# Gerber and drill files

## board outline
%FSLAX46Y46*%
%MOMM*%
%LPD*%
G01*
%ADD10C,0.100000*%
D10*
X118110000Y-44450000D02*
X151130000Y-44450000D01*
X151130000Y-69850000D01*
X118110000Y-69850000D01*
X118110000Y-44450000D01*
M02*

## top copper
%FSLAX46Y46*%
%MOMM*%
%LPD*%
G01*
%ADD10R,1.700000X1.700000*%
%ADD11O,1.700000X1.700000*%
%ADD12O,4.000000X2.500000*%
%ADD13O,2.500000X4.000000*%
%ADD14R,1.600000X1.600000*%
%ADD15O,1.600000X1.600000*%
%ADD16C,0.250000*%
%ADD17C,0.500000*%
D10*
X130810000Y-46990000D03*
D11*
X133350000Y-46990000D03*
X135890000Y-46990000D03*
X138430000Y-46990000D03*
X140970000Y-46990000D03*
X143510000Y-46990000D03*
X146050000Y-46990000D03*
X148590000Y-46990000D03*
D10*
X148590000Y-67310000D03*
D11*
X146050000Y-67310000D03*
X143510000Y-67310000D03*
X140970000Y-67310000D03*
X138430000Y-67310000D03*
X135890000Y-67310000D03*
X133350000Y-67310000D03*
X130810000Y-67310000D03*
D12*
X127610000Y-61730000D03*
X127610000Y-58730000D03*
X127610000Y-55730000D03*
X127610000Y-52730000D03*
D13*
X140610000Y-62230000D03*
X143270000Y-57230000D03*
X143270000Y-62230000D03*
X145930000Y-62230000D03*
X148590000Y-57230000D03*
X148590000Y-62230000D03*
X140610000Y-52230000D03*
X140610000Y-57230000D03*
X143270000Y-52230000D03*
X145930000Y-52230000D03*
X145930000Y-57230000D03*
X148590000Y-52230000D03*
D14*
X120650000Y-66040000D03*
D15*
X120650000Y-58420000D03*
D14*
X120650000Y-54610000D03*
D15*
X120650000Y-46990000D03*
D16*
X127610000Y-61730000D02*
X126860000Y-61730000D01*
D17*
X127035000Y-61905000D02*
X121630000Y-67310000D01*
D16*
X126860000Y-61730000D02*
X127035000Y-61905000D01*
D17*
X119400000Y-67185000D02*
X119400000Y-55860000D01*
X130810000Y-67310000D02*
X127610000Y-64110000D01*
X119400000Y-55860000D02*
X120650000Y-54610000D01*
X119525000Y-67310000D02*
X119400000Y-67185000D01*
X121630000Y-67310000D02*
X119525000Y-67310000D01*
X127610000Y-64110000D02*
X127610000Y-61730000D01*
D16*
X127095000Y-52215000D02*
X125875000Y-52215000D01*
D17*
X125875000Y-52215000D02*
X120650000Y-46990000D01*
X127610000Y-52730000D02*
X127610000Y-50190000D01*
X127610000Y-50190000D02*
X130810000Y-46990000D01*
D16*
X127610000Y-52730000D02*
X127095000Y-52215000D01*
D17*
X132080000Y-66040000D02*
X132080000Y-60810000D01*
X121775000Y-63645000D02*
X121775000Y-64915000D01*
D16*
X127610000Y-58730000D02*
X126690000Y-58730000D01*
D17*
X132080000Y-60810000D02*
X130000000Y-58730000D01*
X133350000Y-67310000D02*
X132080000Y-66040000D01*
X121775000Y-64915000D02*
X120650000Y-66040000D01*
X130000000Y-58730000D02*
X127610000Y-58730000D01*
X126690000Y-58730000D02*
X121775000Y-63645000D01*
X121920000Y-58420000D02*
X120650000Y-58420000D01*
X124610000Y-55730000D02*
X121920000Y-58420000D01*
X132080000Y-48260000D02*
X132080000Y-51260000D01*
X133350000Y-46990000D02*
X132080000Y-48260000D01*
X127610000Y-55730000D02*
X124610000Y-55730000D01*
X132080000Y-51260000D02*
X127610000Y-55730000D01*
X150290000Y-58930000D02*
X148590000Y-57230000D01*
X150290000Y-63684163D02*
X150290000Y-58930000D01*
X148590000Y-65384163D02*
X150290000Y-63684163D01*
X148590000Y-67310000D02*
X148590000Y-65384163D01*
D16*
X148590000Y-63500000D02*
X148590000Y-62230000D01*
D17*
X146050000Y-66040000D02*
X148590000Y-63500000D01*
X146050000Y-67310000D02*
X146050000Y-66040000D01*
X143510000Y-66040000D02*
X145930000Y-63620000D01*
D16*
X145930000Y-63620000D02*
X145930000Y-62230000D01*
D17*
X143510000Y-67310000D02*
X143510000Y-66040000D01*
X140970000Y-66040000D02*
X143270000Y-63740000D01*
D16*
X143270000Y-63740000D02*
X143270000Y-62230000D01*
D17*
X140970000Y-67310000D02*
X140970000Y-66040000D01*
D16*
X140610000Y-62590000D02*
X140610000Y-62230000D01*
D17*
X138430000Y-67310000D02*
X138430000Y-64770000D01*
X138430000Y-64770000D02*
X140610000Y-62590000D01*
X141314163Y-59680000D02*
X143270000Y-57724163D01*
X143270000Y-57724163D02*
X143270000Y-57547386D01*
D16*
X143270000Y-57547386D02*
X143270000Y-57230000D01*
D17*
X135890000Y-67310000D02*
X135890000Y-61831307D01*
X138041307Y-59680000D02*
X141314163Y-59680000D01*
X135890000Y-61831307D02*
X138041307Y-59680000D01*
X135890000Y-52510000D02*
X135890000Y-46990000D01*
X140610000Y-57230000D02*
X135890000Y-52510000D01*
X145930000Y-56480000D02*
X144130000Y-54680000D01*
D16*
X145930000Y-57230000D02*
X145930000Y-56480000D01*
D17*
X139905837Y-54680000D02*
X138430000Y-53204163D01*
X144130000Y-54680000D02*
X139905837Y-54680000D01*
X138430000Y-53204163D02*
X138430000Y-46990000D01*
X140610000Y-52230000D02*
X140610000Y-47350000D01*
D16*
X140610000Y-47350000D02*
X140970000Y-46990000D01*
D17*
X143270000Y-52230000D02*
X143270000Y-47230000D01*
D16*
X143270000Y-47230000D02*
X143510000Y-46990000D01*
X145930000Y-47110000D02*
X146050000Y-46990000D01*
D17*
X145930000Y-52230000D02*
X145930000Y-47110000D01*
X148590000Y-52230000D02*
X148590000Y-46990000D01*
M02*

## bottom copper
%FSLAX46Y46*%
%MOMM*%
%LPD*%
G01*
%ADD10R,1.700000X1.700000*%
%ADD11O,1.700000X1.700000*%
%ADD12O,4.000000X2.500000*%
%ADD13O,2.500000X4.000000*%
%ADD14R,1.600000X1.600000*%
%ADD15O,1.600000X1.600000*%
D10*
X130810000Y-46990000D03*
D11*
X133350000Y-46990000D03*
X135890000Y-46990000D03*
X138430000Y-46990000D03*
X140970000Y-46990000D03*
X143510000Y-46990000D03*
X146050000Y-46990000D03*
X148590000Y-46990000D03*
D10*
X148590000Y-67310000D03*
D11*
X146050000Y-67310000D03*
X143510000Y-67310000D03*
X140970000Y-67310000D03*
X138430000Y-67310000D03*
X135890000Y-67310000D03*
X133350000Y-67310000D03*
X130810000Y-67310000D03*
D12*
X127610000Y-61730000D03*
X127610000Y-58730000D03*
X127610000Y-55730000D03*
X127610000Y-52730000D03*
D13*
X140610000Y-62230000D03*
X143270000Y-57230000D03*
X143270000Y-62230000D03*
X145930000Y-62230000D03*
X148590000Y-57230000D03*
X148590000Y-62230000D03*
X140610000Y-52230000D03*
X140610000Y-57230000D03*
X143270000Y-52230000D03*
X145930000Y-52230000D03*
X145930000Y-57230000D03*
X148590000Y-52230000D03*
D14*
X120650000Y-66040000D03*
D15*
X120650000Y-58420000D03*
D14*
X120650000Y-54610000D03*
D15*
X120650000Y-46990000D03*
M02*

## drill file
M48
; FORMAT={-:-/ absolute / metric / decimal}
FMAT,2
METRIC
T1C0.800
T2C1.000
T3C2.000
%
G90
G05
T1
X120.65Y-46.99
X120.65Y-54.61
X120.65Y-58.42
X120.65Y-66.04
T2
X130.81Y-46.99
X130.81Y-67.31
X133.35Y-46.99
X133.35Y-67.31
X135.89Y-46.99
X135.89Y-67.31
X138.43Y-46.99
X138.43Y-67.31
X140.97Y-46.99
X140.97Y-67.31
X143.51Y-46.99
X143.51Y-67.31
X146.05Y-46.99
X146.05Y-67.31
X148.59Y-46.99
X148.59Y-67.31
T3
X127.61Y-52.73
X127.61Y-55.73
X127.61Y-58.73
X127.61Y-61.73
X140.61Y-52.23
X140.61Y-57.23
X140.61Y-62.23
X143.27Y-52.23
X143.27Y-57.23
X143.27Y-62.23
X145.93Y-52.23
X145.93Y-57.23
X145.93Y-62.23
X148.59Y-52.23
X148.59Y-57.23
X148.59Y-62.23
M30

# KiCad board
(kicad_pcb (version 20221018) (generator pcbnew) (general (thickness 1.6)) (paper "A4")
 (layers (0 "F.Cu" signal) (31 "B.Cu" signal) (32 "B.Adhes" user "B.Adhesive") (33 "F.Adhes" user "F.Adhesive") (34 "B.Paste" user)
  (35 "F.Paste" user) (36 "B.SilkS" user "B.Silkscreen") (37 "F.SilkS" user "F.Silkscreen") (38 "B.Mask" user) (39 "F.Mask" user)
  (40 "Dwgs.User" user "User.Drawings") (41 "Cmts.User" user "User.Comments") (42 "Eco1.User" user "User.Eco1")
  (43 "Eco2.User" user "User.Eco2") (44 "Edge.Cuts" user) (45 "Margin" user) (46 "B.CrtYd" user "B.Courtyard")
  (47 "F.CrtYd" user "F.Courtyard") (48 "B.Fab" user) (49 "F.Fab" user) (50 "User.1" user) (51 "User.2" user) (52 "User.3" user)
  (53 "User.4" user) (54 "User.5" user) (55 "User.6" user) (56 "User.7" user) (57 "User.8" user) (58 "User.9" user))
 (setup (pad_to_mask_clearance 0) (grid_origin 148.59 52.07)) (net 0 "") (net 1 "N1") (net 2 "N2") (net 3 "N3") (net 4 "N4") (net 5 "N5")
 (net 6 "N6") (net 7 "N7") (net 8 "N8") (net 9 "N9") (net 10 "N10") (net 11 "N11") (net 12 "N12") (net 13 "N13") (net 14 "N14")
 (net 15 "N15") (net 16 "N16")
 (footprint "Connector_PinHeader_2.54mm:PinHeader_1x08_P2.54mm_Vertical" (layer "F.Cu") (at 130.81 46.99 90)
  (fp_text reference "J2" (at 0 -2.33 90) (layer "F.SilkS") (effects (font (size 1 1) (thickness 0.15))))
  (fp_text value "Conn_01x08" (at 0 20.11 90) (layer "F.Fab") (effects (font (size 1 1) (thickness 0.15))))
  (pad "1" thru_hole rect (at 0 0 90) (size 1.7 1.7) (drill 1) (layers "*.Cu" "*.Mask") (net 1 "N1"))
  (pad "2" thru_hole oval (at 0 2.54 90) (size 1.7 1.7) (drill 1) (layers "*.Cu" "*.Mask") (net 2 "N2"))
  (pad "3" thru_hole oval (at 0 5.08 90) (size 1.7 1.7) (drill 1) (layers "*.Cu" "*.Mask") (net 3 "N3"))
  (pad "4" thru_hole oval (at 0 7.62 90) (size 1.7 1.7) (drill 1) (layers "*.Cu" "*.Mask") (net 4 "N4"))
  (pad "5" thru_hole oval (at 0 10.16 90) (size 1.7 1.7) (drill 1) (layers "*.Cu" "*.Mask") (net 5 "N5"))
  (pad "6" thru_hole oval (at 0 12.7 90) (size 1.7 1.7) (drill 1) (layers "*.Cu" "*.Mask") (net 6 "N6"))
  (pad "7" thru_hole oval (at 0 15.24 90) (size 1.7 1.7) (drill 1) (layers "*.Cu" "*.Mask") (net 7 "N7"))
  (pad "8" thru_hole oval (at 0 17.78 90) (size 1.7 1.7) (drill 1) (layers "*.Cu" "*.Mask") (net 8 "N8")))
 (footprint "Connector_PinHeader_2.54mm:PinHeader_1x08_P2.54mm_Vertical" (layer "F.Cu") (at 148.59 67.31 -90)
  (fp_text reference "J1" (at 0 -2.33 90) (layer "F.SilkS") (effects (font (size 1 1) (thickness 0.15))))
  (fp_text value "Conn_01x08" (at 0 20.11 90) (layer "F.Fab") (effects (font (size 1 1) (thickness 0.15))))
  (pad "1" thru_hole rect (at 0 0 270) (size 1.7 1.7) (drill 1) (layers "*.Cu" "*.Mask") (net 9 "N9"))
  (pad "2" thru_hole oval (at 0 2.54 270) (size 1.7 1.7) (drill 1) (layers "*.Cu" "*.Mask") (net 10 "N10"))
  (pad "3" thru_hole oval (at 0 5.08 270) (size 1.7 1.7) (drill 1) (layers "*.Cu" "*.Mask") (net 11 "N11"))
  (pad "4" thru_hole oval (at 0 7.62 270) (size 1.7 1.7) (drill 1) (layers "*.Cu" "*.Mask") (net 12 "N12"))
  (pad "5" thru_hole oval (at 0 10.16 270) (size 1.7 1.7) (drill 1) (layers "*.Cu" "*.Mask") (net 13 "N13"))
  (pad "6" thru_hole oval (at 0 12.7 270) (size 1.7 1.7) (drill 1) (layers "*.Cu" "*.Mask") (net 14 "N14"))
  (pad "7" thru_hole oval (at 0 15.24 270) (size 1.7 1.7) (drill 1) (layers "*.Cu" "*.Mask") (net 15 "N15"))
  (pad "8" thru_hole oval (at 0 17.78 270) (size 1.7 1.7) (drill 1) (layers "*.Cu" "*.Mask") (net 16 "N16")))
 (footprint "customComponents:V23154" (layer "F.Cu") (at 140.61 57.23)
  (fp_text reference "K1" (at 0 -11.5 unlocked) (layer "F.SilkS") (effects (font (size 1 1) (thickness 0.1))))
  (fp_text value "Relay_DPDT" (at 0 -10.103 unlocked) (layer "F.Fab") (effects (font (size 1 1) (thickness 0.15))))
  (pad "1" thru_hole oval (at -13 4.5) (size 4 2.5) (drill 2) (layers "*.Cu" "*.Mask") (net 16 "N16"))
  (pad "2" thru_hole oval (at -13 1.5) (size 4 2.5) (drill 2) (layers "*.Cu" "*.Mask") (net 15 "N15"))
  (pad "3" thru_hole oval (at -13 -1.5) (size 4 2.5) (drill 2) (layers "*.Cu" "*.Mask") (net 2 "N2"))
  (pad "4" thru_hole oval (at -13 -4.5) (size 4 2.5) (drill 2) (layers "*.Cu" "*.Mask") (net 1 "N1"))
  (pad "5" thru_hole oval (at 0 5 90) (size 4 2.5) (drill 2) (layers "*.Cu" "*.Mask") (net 13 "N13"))
  (pad "6" thru_hole oval (at 2.66 0 90) (size 4 2.5) (drill 2) (layers "*.Cu" "*.Mask") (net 14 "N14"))
  (pad "7" thru_hole oval (at 2.66 5 90) (size 4 2.5) (drill 2) (layers "*.Cu" "*.Mask") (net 12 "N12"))
  (pad "8" thru_hole oval (at 5.32 5 90) (size 4 2.5) (drill 2) (layers "*.Cu" "*.Mask") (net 11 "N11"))
  (pad "9" thru_hole oval (at 7.98 0 90) (size 4 2.5) (drill 2) (layers "*.Cu" "*.Mask") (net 9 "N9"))
  (pad "10" thru_hole oval (at 7.98 5 90) (size 4 2.5) (drill 2) (layers "*.Cu" "*.Mask") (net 10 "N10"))
  (pad "11" thru_hole oval (at 0 -5 90) (size 4 2.5) (drill 2) (layers "*.Cu" "*.Mask") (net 5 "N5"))
  (pad "12" thru_hole oval (at 0 0 90) (size 4 2.5) (drill 2) (layers "*.Cu" "*.Mask") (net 3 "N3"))
  (pad "13" thru_hole oval (at 2.66 -5 90) (size 4 2.5) (drill 2) (layers "*.Cu" "*.Mask") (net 6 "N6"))
  (pad "14" thru_hole oval (at 5.32 -5 90) (size 4 2.5) (drill 2) (layers "*.Cu" "*.Mask") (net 7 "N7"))
  (pad "15" thru_hole oval (at 5.32 0 90) (size 4 2.5) (drill 2) (layers "*.Cu" "*.Mask") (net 4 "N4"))
  (pad "16" thru_hole oval (at 7.98 -5 90) (size 4 2.5) (drill 2) (layers "*.Cu" "*.Mask") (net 8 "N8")))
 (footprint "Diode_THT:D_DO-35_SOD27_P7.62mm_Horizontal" (layer "F.Cu") (at 120.65 66.04 90)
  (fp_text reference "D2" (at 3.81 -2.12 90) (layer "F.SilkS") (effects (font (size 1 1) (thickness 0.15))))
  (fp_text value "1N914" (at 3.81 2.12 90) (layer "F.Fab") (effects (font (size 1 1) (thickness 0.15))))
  (pad "1" thru_hole rect (at 0 0 90) (size 1.6 1.6) (drill 0.8) (layers "*.Cu" "*.Mask") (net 15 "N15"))
  (pad "2" thru_hole oval (at 7.62 0 90) (size 1.6 1.6) (drill 0.8) (layers "*.Cu" "*.Mask") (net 2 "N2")))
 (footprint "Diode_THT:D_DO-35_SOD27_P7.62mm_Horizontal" (layer "F.Cu") (at 120.65 54.61 90)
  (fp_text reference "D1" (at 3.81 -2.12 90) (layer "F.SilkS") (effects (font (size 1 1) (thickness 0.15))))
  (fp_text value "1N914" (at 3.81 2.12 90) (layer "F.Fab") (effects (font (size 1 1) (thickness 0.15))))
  (pad "1" thru_hole rect (at 0 0 90) (size 1.6 1.6) (drill 0.8) (layers "*.Cu" "*.Mask") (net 16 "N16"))
  (pad "2" thru_hole oval (at 7.62 0 90) (size 1.6 1.6) (drill 0.8) (layers "*.Cu" "*.Mask") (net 1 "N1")))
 (gr_rect (start 118.11 44.45) (end 151.13 69.85) (stroke (width 0.1) (type default)) (fill none) (layer "Edge.Cuts"))
 (segment (start 127.61 61.73) (end 126.86 61.73) (width 0.25) (layer "F.Cu") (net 16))
 (segment (start 127.035 61.905) (end 121.63 67.31) (width 0.5) (layer "F.Cu") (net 16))
 (segment (start 126.86 61.73) (end 127.035 61.905) (width 0.25) (layer "F.Cu") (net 16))
 (segment (start 119.4 67.185) (end 119.4 55.86) (width 0.5) (layer "F.Cu") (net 16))
 (segment (start 130.81 67.31) (end 127.61 64.11) (width 0.5) (layer "F.Cu") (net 16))
 (segment (start 119.4 55.86) (end 120.65 54.61) (width 0.5) (layer "F.Cu") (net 16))
 (segment (start 119.525 67.31) (end 119.4 67.185) (width 0.5) (layer "F.Cu") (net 16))
 (segment (start 121.63 67.31) (end 119.525 67.31) (width 0.5) (layer "F.Cu") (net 16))
 (segment (start 127.61 64.11) (end 127.61 61.73) (width 0.5) (layer "F.Cu") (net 16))
 (segment (start 127.095 52.215) (end 125.875 52.215) (width 0.25) (layer "F.Cu") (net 1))
 (segment (start 125.875 52.215) (end 120.65 46.99) (width 0.5) (layer "F.Cu") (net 1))
 (segment (start 127.61 52.73) (end 127.61 50.19) (width 0.5) (layer "F.Cu") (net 1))
 (segment (start 127.61 50.19) (end 130.81 46.99) (width 0.5) (layer "F.Cu") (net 1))
 (segment (start 127.61 52.73) (end 127.095 52.215) (width 0.25) (layer "F.Cu") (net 1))
 (segment (start 132.08 66.04) (end 132.08 60.81) (width 0.5) (layer "F.Cu") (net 15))
 (segment (start 121.775 63.645) (end 121.775 64.915) (width 0.5) (layer "F.Cu") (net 15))
 (segment (start 127.61 58.73) (end 126.69 58.73) (width 0.25) (layer "F.Cu") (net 15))
 (segment (start 132.08 60.81) (end 130 58.73) (width 0.5) (layer "F.Cu") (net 15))
 (segment (start 133.35 67.31) (end 132.08 66.04) (width 0.5) (layer "F.Cu") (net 15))
 (segment (start 121.775 64.915) (end 120.65 66.04) (width 0.5) (layer "F.Cu") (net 15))
 (segment (start 130 58.73) (end 127.61 58.73) (width 0.5) (layer "F.Cu") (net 15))
 (segment (start 126.69 58.73) (end 121.775 63.645) (width 0.5) (layer "F.Cu") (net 15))
 (segment (start 121.92 58.42) (end 120.65 58.42) (width 0.5) (layer "F.Cu") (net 2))
 (segment (start 124.61 55.73) (end 121.92 58.42) (width 0.5) (layer "F.Cu") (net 2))
 (segment (start 132.08 48.26) (end 132.08 51.26) (width 0.5) (layer "F.Cu") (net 2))
 (segment (start 133.35 46.99) (end 132.08 48.26) (width 0.5) (layer "F.Cu") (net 2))
 (segment (start 127.61 55.73) (end 124.61 55.73) (width 0.5) (layer "F.Cu") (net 2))
 (segment (start 132.08 51.26) (end 127.61 55.73) (width 0.5) (layer "F.Cu") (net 2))
 (segment (start 150.29 58.93) (end 148.59 57.23) (width 0.5) (layer "F.Cu") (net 9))
 (segment (start 150.29 63.684163) (end 150.29 58.93) (width 0.5) (layer "F.Cu") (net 9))
 (segment (start 148.59 65.384163) (end 150.29 63.684163) (width 0.5) (layer "F.Cu") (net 9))
 (segment (start 148.59 67.31) (end 148.59 65.384163) (width 0.5) (layer "F.Cu") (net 9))
 (segment (start 148.59 63.5) (end 148.59 62.23) (width 0.25) (layer "F.Cu") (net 10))
 (segment (start 146.05 66.04) (end 148.59 63.5) (width 0.5) (layer "F.Cu") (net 10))
 (segment (start 146.05 67.31) (end 146.05 66.04) (width 0.5) (layer "F.Cu") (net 10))
 (segment (start 143.51 66.04) (end 145.93 63.62) (width 0.5) (layer "F.Cu") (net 11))
 (segment (start 145.93 63.62) (end 145.93 62.23) (width 0.25) (layer "F.Cu") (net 11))
 (segment (start 143.51 67.31) (end 143.51 66.04) (width 0.5) (layer "F.Cu") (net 11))
 (segment (start 140.97 66.04) (end 143.27 63.74) (width 0.5) (layer "F.Cu") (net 12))
 (segment (start 143.27 63.74) (end 143.27 62.23) (width 0.25) (layer "F.Cu") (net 12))
 (segment (start 140.97 67.31) (end 140.97 66.04) (width 0.5) (layer "F.Cu") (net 12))
 (segment (start 140.61 62.59) (end 140.61 62.23) (width 0.25) (layer "F.Cu") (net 13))
 (segment (start 138.43 67.31) (end 138.43 64.77) (width 0.5) (layer "F.Cu") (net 13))
 (segment (start 138.43 64.77) (end 140.61 62.59) (width 0.5) (layer "F.Cu") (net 13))
 (segment (start 141.314163 59.68) (end 143.27 57.724163) (width 0.5) (layer "F.Cu") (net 14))
 (segment (start 143.27 57.724163) (end 143.27 57.547386) (width 0.5) (layer "F.Cu") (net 14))
 (segment (start 143.27 57.547386) (end 143.27 57.23) (width 0.25) (layer "F.Cu") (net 14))
 (segment (start 135.89 67.31) (end 135.89 61.831307) (width 0.5) (layer "F.Cu") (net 14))
 (segment (start 138.041307 59.68) (end 141.314163 59.68) (width 0.5) (layer "F.Cu") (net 14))
 (segment (start 135.89 61.831307) (end 138.041307 59.68) (width 0.5) (layer "F.Cu") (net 14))
 (segment (start 135.89 52.51) (end 135.89 46.99) (width 0.5) (layer "F.Cu") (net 3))
 (segment (start 140.61 57.23) (end 135.89 52.51) (width 0.5) (layer "F.Cu") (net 3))
 (segment (start 145.93 56.48) (end 144.13 54.68) (width 0.5) (layer "F.Cu") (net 4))
 (segment (start 145.93 57.23) (end 145.93 56.48) (width 0.25) (layer "F.Cu") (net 4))
 (segment (start 139.905837 54.68) (end 138.43 53.204163) (width 0.5) (layer "F.Cu") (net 4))
 (segment (start 144.13 54.68) (end 139.905837 54.68) (width 0.5) (layer "F.Cu") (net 4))
 (segment (start 138.43 53.204163) (end 138.43 46.99) (width 0.5) (layer "F.Cu") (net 4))
 (segment (start 140.61 52.23) (end 140.61 47.35) (width 0.5) (layer "F.Cu") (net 5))
 (segment (start 140.61 47.35) (end 140.97 46.99) (width 0.25) (layer "F.Cu") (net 5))
 (segment (start 143.27 52.23) (end 143.27 47.23) (width 0.5) (layer "F.Cu") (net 6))
 (segment (start 143.27 47.23) (end 143.51 46.99) (width 0.25) (layer "F.Cu") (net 6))
 (segment (start 145.93 47.11) (end 146.05 46.99) (width 0.25) (layer "F.Cu") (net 7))
 (segment (start 145.93 52.23) (end 145.93 47.11) (width 0.5) (layer "F.Cu") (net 7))
 (segment (start 148.59 52.23) (end 148.59 46.99) (width 0.5) (layer "F.Cu") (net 8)))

